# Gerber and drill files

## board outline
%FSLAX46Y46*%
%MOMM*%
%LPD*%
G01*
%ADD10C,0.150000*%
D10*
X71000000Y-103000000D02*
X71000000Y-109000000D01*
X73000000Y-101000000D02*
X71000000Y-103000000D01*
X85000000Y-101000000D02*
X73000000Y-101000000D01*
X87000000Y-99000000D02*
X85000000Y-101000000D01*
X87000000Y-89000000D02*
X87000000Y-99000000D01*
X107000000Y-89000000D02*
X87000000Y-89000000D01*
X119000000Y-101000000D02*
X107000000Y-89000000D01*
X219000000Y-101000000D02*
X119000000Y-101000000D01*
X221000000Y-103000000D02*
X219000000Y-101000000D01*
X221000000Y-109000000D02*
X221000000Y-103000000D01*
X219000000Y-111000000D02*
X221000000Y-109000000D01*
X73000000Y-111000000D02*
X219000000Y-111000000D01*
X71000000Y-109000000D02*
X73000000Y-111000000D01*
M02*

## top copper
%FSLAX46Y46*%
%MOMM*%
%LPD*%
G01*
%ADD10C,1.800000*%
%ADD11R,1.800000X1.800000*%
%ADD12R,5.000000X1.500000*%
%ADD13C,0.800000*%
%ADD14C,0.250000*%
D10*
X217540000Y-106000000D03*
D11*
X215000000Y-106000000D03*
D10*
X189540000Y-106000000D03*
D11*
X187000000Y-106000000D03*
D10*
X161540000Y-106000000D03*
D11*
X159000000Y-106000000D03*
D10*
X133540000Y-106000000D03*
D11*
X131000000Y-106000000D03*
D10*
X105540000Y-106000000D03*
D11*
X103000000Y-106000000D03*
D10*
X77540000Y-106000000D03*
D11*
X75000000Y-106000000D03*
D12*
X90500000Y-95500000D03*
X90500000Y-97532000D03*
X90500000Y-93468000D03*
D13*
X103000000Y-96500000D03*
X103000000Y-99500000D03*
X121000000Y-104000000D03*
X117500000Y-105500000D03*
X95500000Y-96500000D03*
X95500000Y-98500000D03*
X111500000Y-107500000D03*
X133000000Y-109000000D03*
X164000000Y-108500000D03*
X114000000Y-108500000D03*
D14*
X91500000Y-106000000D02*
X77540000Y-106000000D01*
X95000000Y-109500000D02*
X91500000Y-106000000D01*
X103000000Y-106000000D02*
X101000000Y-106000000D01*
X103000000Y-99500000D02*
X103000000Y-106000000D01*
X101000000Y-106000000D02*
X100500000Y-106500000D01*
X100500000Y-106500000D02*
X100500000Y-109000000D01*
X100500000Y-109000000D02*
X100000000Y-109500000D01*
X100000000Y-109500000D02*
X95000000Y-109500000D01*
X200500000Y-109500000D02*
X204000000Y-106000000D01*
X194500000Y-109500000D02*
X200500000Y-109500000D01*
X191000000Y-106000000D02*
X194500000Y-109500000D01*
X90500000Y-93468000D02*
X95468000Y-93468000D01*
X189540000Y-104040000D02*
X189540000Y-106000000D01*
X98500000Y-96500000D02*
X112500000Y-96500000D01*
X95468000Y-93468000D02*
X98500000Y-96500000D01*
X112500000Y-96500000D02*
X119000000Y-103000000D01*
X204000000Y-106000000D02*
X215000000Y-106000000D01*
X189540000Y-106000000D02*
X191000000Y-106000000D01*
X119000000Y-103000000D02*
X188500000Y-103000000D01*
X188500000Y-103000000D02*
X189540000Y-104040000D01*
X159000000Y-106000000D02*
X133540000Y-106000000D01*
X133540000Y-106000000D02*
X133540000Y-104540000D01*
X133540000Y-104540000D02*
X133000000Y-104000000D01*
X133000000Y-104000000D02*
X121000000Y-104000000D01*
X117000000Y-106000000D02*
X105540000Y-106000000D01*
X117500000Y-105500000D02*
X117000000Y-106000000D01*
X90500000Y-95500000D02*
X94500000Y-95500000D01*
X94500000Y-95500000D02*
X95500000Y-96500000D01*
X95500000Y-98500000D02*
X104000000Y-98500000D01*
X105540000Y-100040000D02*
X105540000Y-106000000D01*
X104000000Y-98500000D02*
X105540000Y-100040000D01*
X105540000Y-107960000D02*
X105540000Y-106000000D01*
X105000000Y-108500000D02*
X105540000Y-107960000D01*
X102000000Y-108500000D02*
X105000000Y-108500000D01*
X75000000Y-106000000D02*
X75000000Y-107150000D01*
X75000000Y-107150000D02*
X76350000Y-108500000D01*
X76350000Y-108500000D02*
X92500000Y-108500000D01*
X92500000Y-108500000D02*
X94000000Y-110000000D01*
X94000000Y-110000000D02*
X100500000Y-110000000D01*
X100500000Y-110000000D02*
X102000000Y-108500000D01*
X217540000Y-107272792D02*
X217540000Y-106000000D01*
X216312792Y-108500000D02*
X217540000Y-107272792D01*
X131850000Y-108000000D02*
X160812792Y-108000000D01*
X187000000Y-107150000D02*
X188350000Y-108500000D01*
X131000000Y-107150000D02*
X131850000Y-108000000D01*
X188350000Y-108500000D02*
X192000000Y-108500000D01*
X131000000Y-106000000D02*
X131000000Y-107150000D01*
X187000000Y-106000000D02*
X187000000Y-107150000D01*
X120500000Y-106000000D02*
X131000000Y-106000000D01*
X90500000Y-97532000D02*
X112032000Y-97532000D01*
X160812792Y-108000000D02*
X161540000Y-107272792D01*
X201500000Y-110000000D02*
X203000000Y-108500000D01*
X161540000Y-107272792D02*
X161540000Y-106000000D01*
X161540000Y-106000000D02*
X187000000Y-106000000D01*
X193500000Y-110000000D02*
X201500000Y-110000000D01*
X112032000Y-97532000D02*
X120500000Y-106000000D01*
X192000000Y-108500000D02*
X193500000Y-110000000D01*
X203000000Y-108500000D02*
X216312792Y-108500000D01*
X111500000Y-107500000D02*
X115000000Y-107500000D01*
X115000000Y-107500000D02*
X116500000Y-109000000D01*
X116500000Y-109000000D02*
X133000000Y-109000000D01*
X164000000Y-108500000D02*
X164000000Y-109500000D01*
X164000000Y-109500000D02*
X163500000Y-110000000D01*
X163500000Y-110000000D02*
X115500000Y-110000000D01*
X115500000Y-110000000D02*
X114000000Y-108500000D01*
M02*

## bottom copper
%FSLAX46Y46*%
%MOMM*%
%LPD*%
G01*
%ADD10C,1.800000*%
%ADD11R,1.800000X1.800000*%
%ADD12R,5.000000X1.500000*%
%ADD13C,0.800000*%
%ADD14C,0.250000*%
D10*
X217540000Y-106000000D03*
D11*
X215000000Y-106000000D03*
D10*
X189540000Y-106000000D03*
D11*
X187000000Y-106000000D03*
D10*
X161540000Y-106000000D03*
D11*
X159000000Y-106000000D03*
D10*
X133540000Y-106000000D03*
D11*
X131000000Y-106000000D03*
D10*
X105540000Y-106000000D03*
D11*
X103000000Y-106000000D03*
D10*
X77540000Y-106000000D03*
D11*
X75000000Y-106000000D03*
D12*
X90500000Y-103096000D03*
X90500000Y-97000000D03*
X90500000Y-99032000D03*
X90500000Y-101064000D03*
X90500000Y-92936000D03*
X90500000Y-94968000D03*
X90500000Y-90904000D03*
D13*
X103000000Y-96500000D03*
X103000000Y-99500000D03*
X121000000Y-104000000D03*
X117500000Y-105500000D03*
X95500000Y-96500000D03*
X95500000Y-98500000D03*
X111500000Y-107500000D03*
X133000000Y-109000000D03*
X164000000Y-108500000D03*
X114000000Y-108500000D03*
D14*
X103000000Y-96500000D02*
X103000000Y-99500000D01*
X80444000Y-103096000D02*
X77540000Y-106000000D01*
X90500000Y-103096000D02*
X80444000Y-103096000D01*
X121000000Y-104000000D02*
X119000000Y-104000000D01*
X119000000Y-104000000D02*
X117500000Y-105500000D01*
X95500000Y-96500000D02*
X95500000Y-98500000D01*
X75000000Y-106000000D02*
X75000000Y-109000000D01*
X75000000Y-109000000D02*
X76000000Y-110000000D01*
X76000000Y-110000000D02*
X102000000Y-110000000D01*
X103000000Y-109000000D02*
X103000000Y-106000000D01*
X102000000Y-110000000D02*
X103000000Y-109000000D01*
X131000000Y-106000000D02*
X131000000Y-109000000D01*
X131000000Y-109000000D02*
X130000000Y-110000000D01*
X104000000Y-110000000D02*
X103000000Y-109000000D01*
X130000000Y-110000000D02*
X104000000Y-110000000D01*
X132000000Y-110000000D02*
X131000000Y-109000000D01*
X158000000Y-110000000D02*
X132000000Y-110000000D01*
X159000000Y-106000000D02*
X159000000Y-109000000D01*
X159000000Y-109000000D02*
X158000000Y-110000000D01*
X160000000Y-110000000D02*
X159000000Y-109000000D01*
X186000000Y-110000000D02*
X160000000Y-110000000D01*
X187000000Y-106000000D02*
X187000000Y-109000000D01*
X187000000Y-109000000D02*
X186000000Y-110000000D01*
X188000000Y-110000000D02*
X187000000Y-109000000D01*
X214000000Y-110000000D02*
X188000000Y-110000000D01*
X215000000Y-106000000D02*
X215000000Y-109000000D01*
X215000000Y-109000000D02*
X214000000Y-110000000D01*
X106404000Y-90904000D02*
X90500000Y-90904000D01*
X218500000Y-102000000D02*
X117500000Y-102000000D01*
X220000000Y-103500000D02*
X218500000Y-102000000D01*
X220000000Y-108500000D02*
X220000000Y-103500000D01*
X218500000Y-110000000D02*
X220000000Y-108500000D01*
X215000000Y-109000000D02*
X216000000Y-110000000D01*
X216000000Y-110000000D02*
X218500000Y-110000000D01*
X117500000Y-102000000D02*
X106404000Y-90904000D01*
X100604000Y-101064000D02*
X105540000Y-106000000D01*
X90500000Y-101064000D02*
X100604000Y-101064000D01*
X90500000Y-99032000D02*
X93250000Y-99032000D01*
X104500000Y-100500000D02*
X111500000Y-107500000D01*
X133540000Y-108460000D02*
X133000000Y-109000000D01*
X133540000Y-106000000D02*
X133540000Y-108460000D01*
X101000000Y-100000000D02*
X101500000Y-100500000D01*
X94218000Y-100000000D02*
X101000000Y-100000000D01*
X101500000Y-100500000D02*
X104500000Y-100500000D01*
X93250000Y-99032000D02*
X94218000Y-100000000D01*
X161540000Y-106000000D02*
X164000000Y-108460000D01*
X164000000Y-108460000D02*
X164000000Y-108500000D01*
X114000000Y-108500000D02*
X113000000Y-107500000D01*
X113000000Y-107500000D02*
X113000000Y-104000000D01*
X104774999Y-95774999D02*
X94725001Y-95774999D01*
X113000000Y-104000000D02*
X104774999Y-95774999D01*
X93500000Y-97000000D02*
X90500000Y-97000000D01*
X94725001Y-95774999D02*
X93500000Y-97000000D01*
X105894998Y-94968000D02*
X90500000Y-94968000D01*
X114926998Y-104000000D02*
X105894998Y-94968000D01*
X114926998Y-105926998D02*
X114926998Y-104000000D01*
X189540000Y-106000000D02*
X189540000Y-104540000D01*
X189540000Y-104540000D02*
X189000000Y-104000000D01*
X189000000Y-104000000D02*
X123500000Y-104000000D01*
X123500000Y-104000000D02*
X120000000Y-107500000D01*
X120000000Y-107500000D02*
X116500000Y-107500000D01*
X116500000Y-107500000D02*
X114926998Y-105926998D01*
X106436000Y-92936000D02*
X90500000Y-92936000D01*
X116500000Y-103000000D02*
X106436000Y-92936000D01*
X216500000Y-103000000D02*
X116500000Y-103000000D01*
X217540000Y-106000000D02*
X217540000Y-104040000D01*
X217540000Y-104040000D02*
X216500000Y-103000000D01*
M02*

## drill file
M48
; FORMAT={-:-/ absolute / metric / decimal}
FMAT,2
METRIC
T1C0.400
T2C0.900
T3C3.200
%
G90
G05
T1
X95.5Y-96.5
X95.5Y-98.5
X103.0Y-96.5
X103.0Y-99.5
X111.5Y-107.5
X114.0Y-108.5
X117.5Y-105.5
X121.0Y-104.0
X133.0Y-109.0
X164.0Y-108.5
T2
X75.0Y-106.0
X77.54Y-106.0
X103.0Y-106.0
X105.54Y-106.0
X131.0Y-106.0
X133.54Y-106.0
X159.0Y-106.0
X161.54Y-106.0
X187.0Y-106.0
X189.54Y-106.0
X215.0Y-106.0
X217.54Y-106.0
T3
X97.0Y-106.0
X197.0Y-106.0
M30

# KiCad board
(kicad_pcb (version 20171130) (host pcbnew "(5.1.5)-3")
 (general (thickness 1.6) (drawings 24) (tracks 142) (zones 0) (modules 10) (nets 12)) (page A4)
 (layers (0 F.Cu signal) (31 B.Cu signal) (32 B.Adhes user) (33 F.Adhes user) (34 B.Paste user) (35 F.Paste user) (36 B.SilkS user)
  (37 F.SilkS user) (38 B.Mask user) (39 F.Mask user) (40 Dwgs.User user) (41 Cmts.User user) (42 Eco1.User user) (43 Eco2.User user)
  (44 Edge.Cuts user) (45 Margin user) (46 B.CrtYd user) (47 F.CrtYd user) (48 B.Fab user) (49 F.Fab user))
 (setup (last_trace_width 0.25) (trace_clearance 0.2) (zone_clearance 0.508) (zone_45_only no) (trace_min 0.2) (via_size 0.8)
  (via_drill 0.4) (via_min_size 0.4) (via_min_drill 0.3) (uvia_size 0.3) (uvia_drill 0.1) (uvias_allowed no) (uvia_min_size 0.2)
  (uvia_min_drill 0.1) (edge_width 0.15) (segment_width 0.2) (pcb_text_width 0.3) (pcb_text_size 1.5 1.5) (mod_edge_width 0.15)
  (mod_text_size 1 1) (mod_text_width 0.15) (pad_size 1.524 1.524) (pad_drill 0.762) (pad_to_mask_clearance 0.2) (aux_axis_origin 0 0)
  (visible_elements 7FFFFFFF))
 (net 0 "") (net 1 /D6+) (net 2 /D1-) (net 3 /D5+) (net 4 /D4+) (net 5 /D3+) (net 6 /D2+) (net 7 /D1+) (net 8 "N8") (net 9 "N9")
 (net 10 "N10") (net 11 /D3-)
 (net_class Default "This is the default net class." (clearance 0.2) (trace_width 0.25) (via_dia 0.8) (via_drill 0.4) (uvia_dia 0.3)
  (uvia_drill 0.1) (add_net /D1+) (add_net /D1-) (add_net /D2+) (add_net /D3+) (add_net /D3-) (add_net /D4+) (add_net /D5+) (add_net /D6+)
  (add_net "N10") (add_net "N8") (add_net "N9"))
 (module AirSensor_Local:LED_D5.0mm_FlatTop (layer F.Cu) (at 215 106)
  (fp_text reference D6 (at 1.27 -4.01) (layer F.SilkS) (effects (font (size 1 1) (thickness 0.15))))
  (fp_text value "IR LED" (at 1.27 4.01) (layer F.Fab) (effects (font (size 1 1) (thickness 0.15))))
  (pad 2 thru_hole circle (at 2.54 0) (size 1.8 1.8) (drill 0.9) (layers *.Cu *.Mask) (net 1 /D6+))
  (pad 1 thru_hole rect (at 0 0) (size 1.8 1.8) (drill 0.9) (layers *.Cu *.Mask) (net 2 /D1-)))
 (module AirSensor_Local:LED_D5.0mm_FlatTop (layer F.Cu) (at 187 106)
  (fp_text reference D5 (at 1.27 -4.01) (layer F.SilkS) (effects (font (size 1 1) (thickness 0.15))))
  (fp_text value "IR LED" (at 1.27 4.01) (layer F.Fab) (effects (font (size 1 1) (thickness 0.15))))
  (pad 2 thru_hole circle (at 2.54 0) (size 1.8 1.8) (drill 0.9) (layers *.Cu *.Mask) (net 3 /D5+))
  (pad 1 thru_hole rect (at 0 0) (size 1.8 1.8) (drill 0.9) (layers *.Cu *.Mask) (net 2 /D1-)))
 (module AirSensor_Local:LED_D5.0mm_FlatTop (layer F.Cu) (at 159 106)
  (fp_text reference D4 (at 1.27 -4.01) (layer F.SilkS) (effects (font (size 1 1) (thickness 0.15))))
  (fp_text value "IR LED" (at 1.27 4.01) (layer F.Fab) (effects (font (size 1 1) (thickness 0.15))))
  (pad 2 thru_hole circle (at 2.54 0) (size 1.8 1.8) (drill 0.9) (layers *.Cu *.Mask) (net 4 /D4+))
  (pad 1 thru_hole rect (at 0 0) (size 1.8 1.8) (drill 0.9) (layers *.Cu *.Mask) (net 2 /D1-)))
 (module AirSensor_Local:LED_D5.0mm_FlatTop (layer F.Cu) (at 131 106)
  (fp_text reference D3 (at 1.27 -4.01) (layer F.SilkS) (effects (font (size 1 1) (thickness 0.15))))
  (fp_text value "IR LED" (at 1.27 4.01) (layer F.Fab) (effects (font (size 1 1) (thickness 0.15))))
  (pad 2 thru_hole circle (at 2.54 0) (size 1.8 1.8) (drill 0.9) (layers *.Cu *.Mask) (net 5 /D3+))
  (pad 1 thru_hole rect (at 0 0) (size 1.8 1.8) (drill 0.9) (layers *.Cu *.Mask) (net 2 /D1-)))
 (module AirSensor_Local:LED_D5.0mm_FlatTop (layer F.Cu) (at 103 106)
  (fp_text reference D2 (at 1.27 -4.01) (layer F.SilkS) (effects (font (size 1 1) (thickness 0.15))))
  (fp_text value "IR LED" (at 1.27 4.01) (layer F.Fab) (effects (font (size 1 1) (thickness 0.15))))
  (pad 2 thru_hole circle (at 2.54 0) (size 1.8 1.8) (drill 0.9) (layers *.Cu *.Mask) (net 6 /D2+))
  (pad 1 thru_hole rect (at 0 0) (size 1.8 1.8) (drill 0.9) (layers *.Cu *.Mask) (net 2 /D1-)))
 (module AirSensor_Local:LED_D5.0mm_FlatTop (layer F.Cu) (at 75 106)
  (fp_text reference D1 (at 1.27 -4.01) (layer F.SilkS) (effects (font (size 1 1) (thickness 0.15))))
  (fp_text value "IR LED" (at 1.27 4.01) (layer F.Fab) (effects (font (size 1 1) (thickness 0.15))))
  (pad 2 thru_hole circle (at 2.54 0) (size 1.8 1.8) (drill 0.9) (layers *.Cu *.Mask) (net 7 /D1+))
  (pad 1 thru_hole rect (at 0 0) (size 1.8 1.8) (drill 0.9) (layers *.Cu *.Mask) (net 2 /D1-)))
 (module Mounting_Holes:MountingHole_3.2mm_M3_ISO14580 (layer F.Cu) (at 197 106)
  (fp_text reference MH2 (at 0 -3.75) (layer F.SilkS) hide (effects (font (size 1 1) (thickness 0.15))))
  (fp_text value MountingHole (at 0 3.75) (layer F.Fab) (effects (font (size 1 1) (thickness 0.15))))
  (pad 1 np_thru_hole circle (at 0 0) (size 3.2 3.2) (drill 3.2) (layers *.Cu *.Mask)))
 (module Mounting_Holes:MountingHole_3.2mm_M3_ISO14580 (layer F.Cu) (at 97 106)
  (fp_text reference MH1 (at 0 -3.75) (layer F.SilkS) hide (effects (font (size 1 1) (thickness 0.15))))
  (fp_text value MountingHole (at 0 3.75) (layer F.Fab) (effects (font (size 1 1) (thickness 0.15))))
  (pad 1 np_thru_hole circle (at 0 0) (size 3.2 3.2) (drill 3.2) (layers *.Cu *.Mask)))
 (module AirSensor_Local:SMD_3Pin (layer F.Cu) (at 90.5 95.5)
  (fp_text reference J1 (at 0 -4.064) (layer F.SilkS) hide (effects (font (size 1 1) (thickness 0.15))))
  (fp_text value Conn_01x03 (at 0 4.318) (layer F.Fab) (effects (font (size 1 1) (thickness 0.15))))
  (pad 2 smd rect (at 0 0) (size 5 1.5) (layers F.Cu F.Paste F.Mask) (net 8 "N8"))
  (pad 3 smd rect (at 0 2.032) (size 5 1.5) (layers F.Cu F.Paste F.Mask) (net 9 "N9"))
  (pad 1 smd rect (at 0 -2.032) (size 5 1.5) (layers F.Cu F.Paste F.Mask) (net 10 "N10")))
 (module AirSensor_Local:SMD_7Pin (layer B.Cu) (at 90.5 97 180)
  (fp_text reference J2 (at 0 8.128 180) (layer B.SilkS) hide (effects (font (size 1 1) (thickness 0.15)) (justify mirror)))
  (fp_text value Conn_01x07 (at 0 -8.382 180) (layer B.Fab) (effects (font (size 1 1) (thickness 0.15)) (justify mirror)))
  (pad 7 smd rect (at 0 -6.096 180) (size 5 1.5) (layers B.Cu B.Paste B.Mask) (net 7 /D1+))
  (pad 4 smd rect (at 0 0 180) (size 5 1.5) (layers B.Cu B.Paste B.Mask) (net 4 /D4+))
  (pad 5 smd rect (at 0 -2.032 180) (size 5 1.5) (layers B.Cu B.Paste B.Mask) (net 5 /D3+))
  (pad 6 smd rect (at 0 -4.064 180) (size 5 1.5) (layers B.Cu B.Paste B.Mask) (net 6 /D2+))
  (pad 2 smd rect (at 0 4.064 180) (size 5 1.5) (layers B.Cu B.Paste B.Mask) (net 1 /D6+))
  (pad 3 smd rect (at 0 2.032 180) (size 5 1.5) (layers B.Cu B.Paste B.Mask) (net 3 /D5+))
  (pad 1 smd rect (at 0 6.096 180) (size 5 1.5) (layers B.Cu B.Paste B.Mask) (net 2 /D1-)))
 (gr_line (start 71 103) (end 71 109) (layer Edge.Cuts) (width 0.15))
 (gr_line (start 73 101) (end 71 103) (layer Edge.Cuts) (width 0.15))
 (gr_line (start 85 101) (end 73 101) (layer Edge.Cuts) (width 0.15))
 (gr_line (start 87 99) (end 85 101) (layer Edge.Cuts) (width 0.15))
 (gr_line (start 87 89) (end 87 99) (layer Edge.Cuts) (width 0.15))
 (gr_line (start 107 89) (end 87 89) (layer Edge.Cuts) (width 0.15))
 (gr_line (start 119 101) (end 107 89) (layer Edge.Cuts) (width 0.15))
 (gr_line (start 219 101) (end 119 101) (layer Edge.Cuts) (width 0.15))
 (gr_line (start 221 103) (end 219 101) (layer Edge.Cuts) (width 0.15))
 (gr_line (start 221 109) (end 221 103) (layer Edge.Cuts) (width 0.15))
 (gr_line (start 219 111) (end 221 109) (layer Edge.Cuts) (width 0.15))
 (gr_line (start 73 111) (end 219 111) (layer Edge.Cuts) (width 0.15))
 (gr_line (start 71 109) (end 73 111) (layer Edge.Cuts) (width 0.15))
 (via (at 103 96.5) (size 0.8) (drill 0.4) (layers F.Cu B.Cu) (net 7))
 (via (at 103 99.5) (size 0.8) (drill 0.4) (layers F.Cu B.Cu) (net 7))
 (segment (start 103 96.5) (end 103 99.5) (width 0.25) (layer B.Cu) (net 7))
 (segment (start 80.444 103.096) (end 77.54 106) (width 0.25) (layer B.Cu) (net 7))
 (segment (start 90.5 103.096) (end 80.444 103.096) (width 0.25) (layer B.Cu) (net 7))
 (segment (start 91.5 106) (end 77.54 106) (width 0.25) (layer F.Cu) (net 7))
 (segment (start 95 109.5) (end 91.5 106) (width 0.25) (layer F.Cu) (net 7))
 (segment (start 103 106) (end 101 106) (width 0.25) (layer F.Cu) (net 7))
 (segment (start 103 99.5) (end 103 106) (width 0.25) (layer F.Cu) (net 7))
 (segment (start 101 106) (end 100.5 106.5) (width 0.25) (layer F.Cu) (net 7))
 (segment (start 100.5 106.5) (end 100.5 109) (width 0.25) (layer F.Cu) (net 7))
 (segment (start 100.5 109) (end 100 109.5) (width 0.25) (layer F.Cu) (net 7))
 (segment (start 100 109.5) (end 95 109.5) (width 0.25) (layer F.Cu) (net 7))
 (segment (start 200.5 109.5) (end 204 106) (width 0.25) (layer F.Cu) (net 7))
 (segment (start 194.5 109.5) (end 200.5 109.5) (width 0.25) (layer F.Cu) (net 7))
 (segment (start 191 106) (end 194.5 109.5) (width 0.25) (layer F.Cu) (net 7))
 (segment (start 90.5 93.468) (end 95.468 93.468) (width 0.25) (layer F.Cu) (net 7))
 (segment (start 189.54 104.04) (end 189.54 106) (width 0.25) (layer F.Cu) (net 7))
 (segment (start 98.5 96.5) (end 112.5 96.5) (width 0.25) (layer F.Cu) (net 7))
 (segment (start 95.468 93.468) (end 98.5 96.5) (width 0.25) (layer F.Cu) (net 7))
 (segment (start 112.5 96.5) (end 119 103) (width 0.25) (layer F.Cu) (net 7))
 (segment (start 204 106) (end 215 106) (width 0.25) (layer F.Cu) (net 7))
 (segment (start 189.54 106) (end 191 106) (width 0.25) (layer F.Cu) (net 7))
 (segment (start 119 103) (end 188.5 103) (width 0.25) (layer F.Cu) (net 7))
 (segment (start 188.5 103) (end 189.54 104.04) (width 0.25) (layer F.Cu) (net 7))
 (segment (start 159 106) (end 133.54 106) (width 0.25) (layer F.Cu) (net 2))
 (segment (start 133.54 106) (end 133.54 104.54) (width 0.25) (layer F.Cu) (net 2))
 (via (at 121 104) (size 0.8) (drill 0.4) (layers F.Cu B.Cu) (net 2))
 (segment (start 133.54 104.54) (end 133 104) (width 0.25) (layer F.Cu) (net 2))
 (segment (start 133 104) (end 121 104) (width 0.25) (layer F.Cu) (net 2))
 (via (at 117.5 105.5) (size 0.8) (drill 0.4) (layers F.Cu B.Cu) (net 2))
 (segment (start 121 104) (end 119 104) (width 0.25) (layer B.Cu) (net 2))
 (segment (start 119 104) (end 117.5 105.5) (width 0.25) (layer B.Cu) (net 2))
 (segment (start 117 106) (end 105.54 106) (width 0.25) (layer F.Cu) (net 2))
 (segment (start 117.5 105.5) (end 117 106) (width 0.25) (layer F.Cu) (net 2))
 (via (at 95.5 96.5) (size 0.8) (drill 0.4) (layers F.Cu B.Cu) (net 2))
 (segment (start 90.5 95.5) (end 94.5 95.5) (width 0.25) (layer F.Cu) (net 2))
 (segment (start 94.5 95.5) (end 95.5 96.5) (width 0.25) (layer F.Cu) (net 2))
 (segment (start 95.5 96.5) (end 95.5 98.5) (width 0.25) (layer B.Cu) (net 2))
 (via (at 95.5 98.5) (size 0.8) (drill 0.4) (layers F.Cu B.Cu) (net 2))
 (segment (start 95.5 98.5) (end 104 98.5) (width 0.25) (layer F.Cu) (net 2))
 (segment (start 105.54 100.04) (end 105.54 106) (width 0.25) (layer F.Cu) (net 2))
 (segment (start 104 98.5) (end 105.54 100.04) (width 0.25) (layer F.Cu) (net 2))
 (segment (start 75 106) (end 75 109) (width 0.25) (layer B.Cu) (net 2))
 (segment (start 75 109) (end 76 110) (width 0.25) (layer B.Cu) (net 2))
 (segment (start 76 110) (end 102 110) (width 0.25) (layer B.Cu) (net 2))
 (segment (start 103 109) (end 103 106) (width 0.25) (layer B.Cu) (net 2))
 (segment (start 102 110) (end 103 109) (width 0.25) (layer B.Cu) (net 2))
 (segment (start 131 106) (end 131 109) (width 0.25) (layer B.Cu) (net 2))
 (segment (start 131 109) (end 130 110) (width 0.25) (layer B.Cu) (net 2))
 (segment (start 104 110) (end 103 109) (width 0.25) (layer B.Cu) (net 2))
 (segment (start 130 110) (end 104 110) (width 0.25) (layer B.Cu) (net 2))
 (segment (start 132 110) (end 131 109) (width 0.25) (layer B.Cu) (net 2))
 (segment (start 158 110) (end 132 110) (width 0.25) (layer B.Cu) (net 2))
 (segment (start 159 106) (end 159 109) (width 0.25) (layer B.Cu) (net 2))
 (segment (start 159 109) (end 158 110) (width 0.25) (layer B.Cu) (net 2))
 (segment (start 160 110) (end 159 109) (width 0.25) (layer B.Cu) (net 2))
 (segment (start 186 110) (end 160 110) (width 0.25) (layer B.Cu) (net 2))
 (segment (start 187 106) (end 187 109) (width 0.25) (layer B.Cu) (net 2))
 (segment (start 187 109) (end 186 110) (width 0.25) (layer B.Cu) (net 2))
 (segment (start 188 110) (end 187 109) (width 0.25) (layer B.Cu) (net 2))
 (segment (start 214 110) (end 188 110) (width 0.25) (layer B.Cu) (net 2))
 (segment (start 215 106) (end 215 109) (width 0.25) (layer B.Cu) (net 2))
 (segment (start 215 109) (end 214 110) (width 0.25) (layer B.Cu) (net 2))
 (segment (start 106.404 90.904) (end 90.5 90.904) (width 0.25) (layer B.Cu) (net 2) (status 1000000))
 (segment (start 218.5 102) (end 117.5 102) (width 0.25) (layer B.Cu) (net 2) (status 1000000))
 (segment (start 220 103.5) (end 218.5 102) (width 0.25) (layer B.Cu) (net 2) (status 1000000))
 (segment (start 220 108.5) (end 220 103.5) (width 0.25) (layer B.Cu) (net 2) (status 1000000))
 (segment (start 218.5 110) (end 220 108.5) (width 0.25) (layer B.Cu) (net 2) (status 1000000))
 (segment (start 215 109) (end 216 110) (width 0.25) (layer B.Cu) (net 2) (status 1000000))
 (segment (start 216 110) (end 218.5 110) (width 0.25) (layer B.Cu) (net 2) (status 1000000))
 (segment (start 117.5 102) (end 106.404 90.904) (width 0.25) (layer B.Cu) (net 2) (status 1000000))
 (segment (start 105.54 107.96) (end 105.54 106) (width 0.25) (layer F.Cu) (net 2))
 (segment (start 105 108.5) (end 105.54 107.96) (width 0.25) (layer F.Cu) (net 2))
 (segment (start 102 108.5) (end 105 108.5) (width 0.25) (layer F.Cu) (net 2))
 (segment (start 75 106) (end 75 107.15) (width 0.25) (layer F.Cu) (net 2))
 (segment (start 75 107.15) (end 76.35 108.5) (width 0.25) (layer F.Cu) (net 2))
 (segment (start 76.35 108.5) (end 92.5 108.5) (width 0.25) (layer F.Cu) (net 2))
 (segment (start 92.5 108.5) (end 94 110) (width 0.25) (layer F.Cu) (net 2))
 (segment (start 94 110) (end 100.5 110) (width 0.25) (layer F.Cu) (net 2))
 (segment (start 100.5 110) (end 102 108.5) (width 0.25) (layer F.Cu) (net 2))
 (segment (start 217.54 107.272792) (end 217.54 106) (width 0.25) (layer F.Cu) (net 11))
 (segment (start 216.312792 108.5) (end 217.54 107.272792) (width 0.25) (layer F.Cu) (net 11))
 (segment (start 131.85 108) (end 160.812792 108) (width 0.25) (layer F.Cu) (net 11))
 (segment (start 187 107.15) (end 188.35 108.5) (width 0.25) (layer F.Cu) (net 11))
 (segment (start 131 107.15) (end 131.85 108) (width 0.25) (layer F.Cu) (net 11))
 (segment (start 188.35 108.5) (end 192 108.5) (width 0.25) (layer F.Cu) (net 11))
 (segment (start 131 106) (end 131 107.15) (width 0.25) (layer F.Cu) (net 11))
 (segment (start 187 106) (end 187 107.15) (width 0.25) (layer F.Cu) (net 11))
 (segment (start 120.5 106) (end 131 106) (width 0.25) (layer F.Cu) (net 11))
 (segment (start 90.5 97.532) (end 112.032 97.532) (width 0.25) (layer F.Cu) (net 11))
 (segment (start 160.812792 108) (end 161.54 107.272792) (width 0.25) (layer F.Cu) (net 11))
 (segment (start 201.5 110) (end 203 108.5) (width 0.25) (layer F.Cu) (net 11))
 (segment (start 161.54 107.272792) (end 161.54 106) (width 0.25) (layer F.Cu) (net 11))
 (segment (start 161.54 106) (end 187 106) (width 0.25) (layer F.Cu) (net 11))
 (segment (start 193.5 110) (end 201.5 110) (width 0.25) (layer F.Cu) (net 11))
 (segment (start 112.032 97.532) (end 120.5 106) (width 0.25) (layer F.Cu) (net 11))
 (segment (start 192 108.5) (end 193.5 110) (width 0.25) (layer F.Cu) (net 11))
 (segment (start 203 108.5) (end 216.312792 108.5) (width 0.25) (layer F.Cu) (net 11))
 (segment (start 100.604 101.064) (end 105.54 106) (width 0.25) (layer B.Cu) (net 6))
 (segment (start 90.5 101.064) (end 100.604 101.064) (width 0.25) (layer B.Cu) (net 6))
 (segment (start 90.5 99.032) (end 93.25 99.032) (width 0.25) (layer B.Cu) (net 5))
 (via (at 111.5 107.5) (size 0.8) (drill 0.4) (layers F.Cu B.Cu) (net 5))
 (segment (start 104.5 100.5) (end 111.5 107.5) (width 0.25) (layer B.Cu) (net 5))
 (segment (start 111.5 107.5) (end 115 107.5) (width 0.25) (layer F.Cu) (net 5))
 (via (at 133 109) (size 0.8) (drill 0.4) (layers F.Cu B.Cu) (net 5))
 (segment (start 115 107.5) (end 116.5 109) (width 0.25) (layer F.Cu) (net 5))
 (segment (start 116.5 109) (end 133 109) (width 0.25) (layer F.Cu) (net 5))
 (segment (start 133.54 108.46) (end 133 109) (width 0.25) (layer B.Cu) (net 5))
 (segment (start 133.54 106) (end 133.54 108.46) (width 0.25) (layer B.Cu) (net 5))
 (segment (start 101 100) (end 101.5 100.5) (width 0.25) (layer B.Cu) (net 5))
 (segment (start 94.218 100) (end 101 100) (width 0.25) (layer B.Cu) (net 5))
 (segment (start 101.5 100.5) (end 104.5 100.5) (width 0.25) (layer B.Cu) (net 5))
 (segment (start 93.25 99.032) (end 94.218 100) (width 0.25) (layer B.Cu) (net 5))
 (via (at 164 108.5) (size 0.8) (drill 0.4) (layers F.Cu B.Cu) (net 4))
 (segment (start 161.54 106) (end 164 108.46) (width 0.25) (layer B.Cu) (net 4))
 (segment (start 164 108.46) (end 164 108.5) (width 0.25) (layer B.Cu) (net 4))
 (segment (start 164 108.5) (end 164 109.5) (width 0.25) (layer F.Cu) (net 4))
 (segment (start 164 109.5) (end 163.5 110) (width 0.25) (layer F.Cu) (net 4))
 (via (at 114 108.5) (size 0.8) (drill 0.4) (layers F.Cu B.Cu) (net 4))
 (segment (start 163.5 110) (end 115.5 110) (width 0.25) (layer F.Cu) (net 4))
 (segment (start 115.5 110) (end 114 108.5) (width 0.25) (layer F.Cu) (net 4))
 (segment (start 114 108.5) (end 113 107.5) (width 0.25) (layer B.Cu) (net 4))
 (segment (start 113 107.5) (end 113 104) (width 0.25) (layer B.Cu) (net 4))
 (segment (start 104.774999 95.774999) (end 94.725001 95.774999) (width 0.25) (layer B.Cu) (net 4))
 (segment (start 113 104) (end 104.774999 95.774999) (width 0.25) (layer B.Cu) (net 4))
 (segment (start 93.5 97) (end 90.5 97) (width 0.25) (layer B.Cu) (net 4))
 (segment (start 94.725001 95.774999) (end 93.5 97) (width 0.25) (layer B.Cu) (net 4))
 (segment (start 105.894998 94.968) (end 90.5 94.968) (width 0.25) (layer B.Cu) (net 3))
 (segment (start 114.926998 104) (end 105.894998 94.968) (width 0.25) (layer B.Cu) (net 3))
 (segment (start 114.926998 105.926998) (end 114.926998 104) (width 0.25) (layer B.Cu) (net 3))
 (segment (start 189.54 106) (end 189.54 104.54) (width 0.25) (layer B.Cu) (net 3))
 (segment (start 189.54 104.54) (end 189 104) (width 0.25) (layer B.Cu) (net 3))
 (segment (start 189 104) (end 123.5 104) (width 0.25) (layer B.Cu) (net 3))
 (segment (start 123.5 104) (end 120 107.5) (width 0.25) (layer B.Cu) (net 3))
 (segment (start 120 107.5) (end 116.5 107.5) (width 0.25) (layer B.Cu) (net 3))
 (segment (start 116.5 107.5) (end 114.926998 105.926998) (width 0.25) (layer B.Cu) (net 3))
 (segment (start 106.436 92.936) (end 90.5 92.936) (width 0.25) (layer B.Cu) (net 1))
 (segment (start 116.5 103) (end 106.436 92.936) (width 0.25) (layer B.Cu) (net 1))
 (segment (start 216.5 103) (end 116.5 103) (width 0.25) (layer B.Cu) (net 1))
 (segment (start 217.54 106) (end 217.54 104.04) (width 0.25) (layer B.Cu) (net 1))
 (segment (start 217.54 104.04) (end 216.5 103) (width 0.25) (layer B.Cu) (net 1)))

